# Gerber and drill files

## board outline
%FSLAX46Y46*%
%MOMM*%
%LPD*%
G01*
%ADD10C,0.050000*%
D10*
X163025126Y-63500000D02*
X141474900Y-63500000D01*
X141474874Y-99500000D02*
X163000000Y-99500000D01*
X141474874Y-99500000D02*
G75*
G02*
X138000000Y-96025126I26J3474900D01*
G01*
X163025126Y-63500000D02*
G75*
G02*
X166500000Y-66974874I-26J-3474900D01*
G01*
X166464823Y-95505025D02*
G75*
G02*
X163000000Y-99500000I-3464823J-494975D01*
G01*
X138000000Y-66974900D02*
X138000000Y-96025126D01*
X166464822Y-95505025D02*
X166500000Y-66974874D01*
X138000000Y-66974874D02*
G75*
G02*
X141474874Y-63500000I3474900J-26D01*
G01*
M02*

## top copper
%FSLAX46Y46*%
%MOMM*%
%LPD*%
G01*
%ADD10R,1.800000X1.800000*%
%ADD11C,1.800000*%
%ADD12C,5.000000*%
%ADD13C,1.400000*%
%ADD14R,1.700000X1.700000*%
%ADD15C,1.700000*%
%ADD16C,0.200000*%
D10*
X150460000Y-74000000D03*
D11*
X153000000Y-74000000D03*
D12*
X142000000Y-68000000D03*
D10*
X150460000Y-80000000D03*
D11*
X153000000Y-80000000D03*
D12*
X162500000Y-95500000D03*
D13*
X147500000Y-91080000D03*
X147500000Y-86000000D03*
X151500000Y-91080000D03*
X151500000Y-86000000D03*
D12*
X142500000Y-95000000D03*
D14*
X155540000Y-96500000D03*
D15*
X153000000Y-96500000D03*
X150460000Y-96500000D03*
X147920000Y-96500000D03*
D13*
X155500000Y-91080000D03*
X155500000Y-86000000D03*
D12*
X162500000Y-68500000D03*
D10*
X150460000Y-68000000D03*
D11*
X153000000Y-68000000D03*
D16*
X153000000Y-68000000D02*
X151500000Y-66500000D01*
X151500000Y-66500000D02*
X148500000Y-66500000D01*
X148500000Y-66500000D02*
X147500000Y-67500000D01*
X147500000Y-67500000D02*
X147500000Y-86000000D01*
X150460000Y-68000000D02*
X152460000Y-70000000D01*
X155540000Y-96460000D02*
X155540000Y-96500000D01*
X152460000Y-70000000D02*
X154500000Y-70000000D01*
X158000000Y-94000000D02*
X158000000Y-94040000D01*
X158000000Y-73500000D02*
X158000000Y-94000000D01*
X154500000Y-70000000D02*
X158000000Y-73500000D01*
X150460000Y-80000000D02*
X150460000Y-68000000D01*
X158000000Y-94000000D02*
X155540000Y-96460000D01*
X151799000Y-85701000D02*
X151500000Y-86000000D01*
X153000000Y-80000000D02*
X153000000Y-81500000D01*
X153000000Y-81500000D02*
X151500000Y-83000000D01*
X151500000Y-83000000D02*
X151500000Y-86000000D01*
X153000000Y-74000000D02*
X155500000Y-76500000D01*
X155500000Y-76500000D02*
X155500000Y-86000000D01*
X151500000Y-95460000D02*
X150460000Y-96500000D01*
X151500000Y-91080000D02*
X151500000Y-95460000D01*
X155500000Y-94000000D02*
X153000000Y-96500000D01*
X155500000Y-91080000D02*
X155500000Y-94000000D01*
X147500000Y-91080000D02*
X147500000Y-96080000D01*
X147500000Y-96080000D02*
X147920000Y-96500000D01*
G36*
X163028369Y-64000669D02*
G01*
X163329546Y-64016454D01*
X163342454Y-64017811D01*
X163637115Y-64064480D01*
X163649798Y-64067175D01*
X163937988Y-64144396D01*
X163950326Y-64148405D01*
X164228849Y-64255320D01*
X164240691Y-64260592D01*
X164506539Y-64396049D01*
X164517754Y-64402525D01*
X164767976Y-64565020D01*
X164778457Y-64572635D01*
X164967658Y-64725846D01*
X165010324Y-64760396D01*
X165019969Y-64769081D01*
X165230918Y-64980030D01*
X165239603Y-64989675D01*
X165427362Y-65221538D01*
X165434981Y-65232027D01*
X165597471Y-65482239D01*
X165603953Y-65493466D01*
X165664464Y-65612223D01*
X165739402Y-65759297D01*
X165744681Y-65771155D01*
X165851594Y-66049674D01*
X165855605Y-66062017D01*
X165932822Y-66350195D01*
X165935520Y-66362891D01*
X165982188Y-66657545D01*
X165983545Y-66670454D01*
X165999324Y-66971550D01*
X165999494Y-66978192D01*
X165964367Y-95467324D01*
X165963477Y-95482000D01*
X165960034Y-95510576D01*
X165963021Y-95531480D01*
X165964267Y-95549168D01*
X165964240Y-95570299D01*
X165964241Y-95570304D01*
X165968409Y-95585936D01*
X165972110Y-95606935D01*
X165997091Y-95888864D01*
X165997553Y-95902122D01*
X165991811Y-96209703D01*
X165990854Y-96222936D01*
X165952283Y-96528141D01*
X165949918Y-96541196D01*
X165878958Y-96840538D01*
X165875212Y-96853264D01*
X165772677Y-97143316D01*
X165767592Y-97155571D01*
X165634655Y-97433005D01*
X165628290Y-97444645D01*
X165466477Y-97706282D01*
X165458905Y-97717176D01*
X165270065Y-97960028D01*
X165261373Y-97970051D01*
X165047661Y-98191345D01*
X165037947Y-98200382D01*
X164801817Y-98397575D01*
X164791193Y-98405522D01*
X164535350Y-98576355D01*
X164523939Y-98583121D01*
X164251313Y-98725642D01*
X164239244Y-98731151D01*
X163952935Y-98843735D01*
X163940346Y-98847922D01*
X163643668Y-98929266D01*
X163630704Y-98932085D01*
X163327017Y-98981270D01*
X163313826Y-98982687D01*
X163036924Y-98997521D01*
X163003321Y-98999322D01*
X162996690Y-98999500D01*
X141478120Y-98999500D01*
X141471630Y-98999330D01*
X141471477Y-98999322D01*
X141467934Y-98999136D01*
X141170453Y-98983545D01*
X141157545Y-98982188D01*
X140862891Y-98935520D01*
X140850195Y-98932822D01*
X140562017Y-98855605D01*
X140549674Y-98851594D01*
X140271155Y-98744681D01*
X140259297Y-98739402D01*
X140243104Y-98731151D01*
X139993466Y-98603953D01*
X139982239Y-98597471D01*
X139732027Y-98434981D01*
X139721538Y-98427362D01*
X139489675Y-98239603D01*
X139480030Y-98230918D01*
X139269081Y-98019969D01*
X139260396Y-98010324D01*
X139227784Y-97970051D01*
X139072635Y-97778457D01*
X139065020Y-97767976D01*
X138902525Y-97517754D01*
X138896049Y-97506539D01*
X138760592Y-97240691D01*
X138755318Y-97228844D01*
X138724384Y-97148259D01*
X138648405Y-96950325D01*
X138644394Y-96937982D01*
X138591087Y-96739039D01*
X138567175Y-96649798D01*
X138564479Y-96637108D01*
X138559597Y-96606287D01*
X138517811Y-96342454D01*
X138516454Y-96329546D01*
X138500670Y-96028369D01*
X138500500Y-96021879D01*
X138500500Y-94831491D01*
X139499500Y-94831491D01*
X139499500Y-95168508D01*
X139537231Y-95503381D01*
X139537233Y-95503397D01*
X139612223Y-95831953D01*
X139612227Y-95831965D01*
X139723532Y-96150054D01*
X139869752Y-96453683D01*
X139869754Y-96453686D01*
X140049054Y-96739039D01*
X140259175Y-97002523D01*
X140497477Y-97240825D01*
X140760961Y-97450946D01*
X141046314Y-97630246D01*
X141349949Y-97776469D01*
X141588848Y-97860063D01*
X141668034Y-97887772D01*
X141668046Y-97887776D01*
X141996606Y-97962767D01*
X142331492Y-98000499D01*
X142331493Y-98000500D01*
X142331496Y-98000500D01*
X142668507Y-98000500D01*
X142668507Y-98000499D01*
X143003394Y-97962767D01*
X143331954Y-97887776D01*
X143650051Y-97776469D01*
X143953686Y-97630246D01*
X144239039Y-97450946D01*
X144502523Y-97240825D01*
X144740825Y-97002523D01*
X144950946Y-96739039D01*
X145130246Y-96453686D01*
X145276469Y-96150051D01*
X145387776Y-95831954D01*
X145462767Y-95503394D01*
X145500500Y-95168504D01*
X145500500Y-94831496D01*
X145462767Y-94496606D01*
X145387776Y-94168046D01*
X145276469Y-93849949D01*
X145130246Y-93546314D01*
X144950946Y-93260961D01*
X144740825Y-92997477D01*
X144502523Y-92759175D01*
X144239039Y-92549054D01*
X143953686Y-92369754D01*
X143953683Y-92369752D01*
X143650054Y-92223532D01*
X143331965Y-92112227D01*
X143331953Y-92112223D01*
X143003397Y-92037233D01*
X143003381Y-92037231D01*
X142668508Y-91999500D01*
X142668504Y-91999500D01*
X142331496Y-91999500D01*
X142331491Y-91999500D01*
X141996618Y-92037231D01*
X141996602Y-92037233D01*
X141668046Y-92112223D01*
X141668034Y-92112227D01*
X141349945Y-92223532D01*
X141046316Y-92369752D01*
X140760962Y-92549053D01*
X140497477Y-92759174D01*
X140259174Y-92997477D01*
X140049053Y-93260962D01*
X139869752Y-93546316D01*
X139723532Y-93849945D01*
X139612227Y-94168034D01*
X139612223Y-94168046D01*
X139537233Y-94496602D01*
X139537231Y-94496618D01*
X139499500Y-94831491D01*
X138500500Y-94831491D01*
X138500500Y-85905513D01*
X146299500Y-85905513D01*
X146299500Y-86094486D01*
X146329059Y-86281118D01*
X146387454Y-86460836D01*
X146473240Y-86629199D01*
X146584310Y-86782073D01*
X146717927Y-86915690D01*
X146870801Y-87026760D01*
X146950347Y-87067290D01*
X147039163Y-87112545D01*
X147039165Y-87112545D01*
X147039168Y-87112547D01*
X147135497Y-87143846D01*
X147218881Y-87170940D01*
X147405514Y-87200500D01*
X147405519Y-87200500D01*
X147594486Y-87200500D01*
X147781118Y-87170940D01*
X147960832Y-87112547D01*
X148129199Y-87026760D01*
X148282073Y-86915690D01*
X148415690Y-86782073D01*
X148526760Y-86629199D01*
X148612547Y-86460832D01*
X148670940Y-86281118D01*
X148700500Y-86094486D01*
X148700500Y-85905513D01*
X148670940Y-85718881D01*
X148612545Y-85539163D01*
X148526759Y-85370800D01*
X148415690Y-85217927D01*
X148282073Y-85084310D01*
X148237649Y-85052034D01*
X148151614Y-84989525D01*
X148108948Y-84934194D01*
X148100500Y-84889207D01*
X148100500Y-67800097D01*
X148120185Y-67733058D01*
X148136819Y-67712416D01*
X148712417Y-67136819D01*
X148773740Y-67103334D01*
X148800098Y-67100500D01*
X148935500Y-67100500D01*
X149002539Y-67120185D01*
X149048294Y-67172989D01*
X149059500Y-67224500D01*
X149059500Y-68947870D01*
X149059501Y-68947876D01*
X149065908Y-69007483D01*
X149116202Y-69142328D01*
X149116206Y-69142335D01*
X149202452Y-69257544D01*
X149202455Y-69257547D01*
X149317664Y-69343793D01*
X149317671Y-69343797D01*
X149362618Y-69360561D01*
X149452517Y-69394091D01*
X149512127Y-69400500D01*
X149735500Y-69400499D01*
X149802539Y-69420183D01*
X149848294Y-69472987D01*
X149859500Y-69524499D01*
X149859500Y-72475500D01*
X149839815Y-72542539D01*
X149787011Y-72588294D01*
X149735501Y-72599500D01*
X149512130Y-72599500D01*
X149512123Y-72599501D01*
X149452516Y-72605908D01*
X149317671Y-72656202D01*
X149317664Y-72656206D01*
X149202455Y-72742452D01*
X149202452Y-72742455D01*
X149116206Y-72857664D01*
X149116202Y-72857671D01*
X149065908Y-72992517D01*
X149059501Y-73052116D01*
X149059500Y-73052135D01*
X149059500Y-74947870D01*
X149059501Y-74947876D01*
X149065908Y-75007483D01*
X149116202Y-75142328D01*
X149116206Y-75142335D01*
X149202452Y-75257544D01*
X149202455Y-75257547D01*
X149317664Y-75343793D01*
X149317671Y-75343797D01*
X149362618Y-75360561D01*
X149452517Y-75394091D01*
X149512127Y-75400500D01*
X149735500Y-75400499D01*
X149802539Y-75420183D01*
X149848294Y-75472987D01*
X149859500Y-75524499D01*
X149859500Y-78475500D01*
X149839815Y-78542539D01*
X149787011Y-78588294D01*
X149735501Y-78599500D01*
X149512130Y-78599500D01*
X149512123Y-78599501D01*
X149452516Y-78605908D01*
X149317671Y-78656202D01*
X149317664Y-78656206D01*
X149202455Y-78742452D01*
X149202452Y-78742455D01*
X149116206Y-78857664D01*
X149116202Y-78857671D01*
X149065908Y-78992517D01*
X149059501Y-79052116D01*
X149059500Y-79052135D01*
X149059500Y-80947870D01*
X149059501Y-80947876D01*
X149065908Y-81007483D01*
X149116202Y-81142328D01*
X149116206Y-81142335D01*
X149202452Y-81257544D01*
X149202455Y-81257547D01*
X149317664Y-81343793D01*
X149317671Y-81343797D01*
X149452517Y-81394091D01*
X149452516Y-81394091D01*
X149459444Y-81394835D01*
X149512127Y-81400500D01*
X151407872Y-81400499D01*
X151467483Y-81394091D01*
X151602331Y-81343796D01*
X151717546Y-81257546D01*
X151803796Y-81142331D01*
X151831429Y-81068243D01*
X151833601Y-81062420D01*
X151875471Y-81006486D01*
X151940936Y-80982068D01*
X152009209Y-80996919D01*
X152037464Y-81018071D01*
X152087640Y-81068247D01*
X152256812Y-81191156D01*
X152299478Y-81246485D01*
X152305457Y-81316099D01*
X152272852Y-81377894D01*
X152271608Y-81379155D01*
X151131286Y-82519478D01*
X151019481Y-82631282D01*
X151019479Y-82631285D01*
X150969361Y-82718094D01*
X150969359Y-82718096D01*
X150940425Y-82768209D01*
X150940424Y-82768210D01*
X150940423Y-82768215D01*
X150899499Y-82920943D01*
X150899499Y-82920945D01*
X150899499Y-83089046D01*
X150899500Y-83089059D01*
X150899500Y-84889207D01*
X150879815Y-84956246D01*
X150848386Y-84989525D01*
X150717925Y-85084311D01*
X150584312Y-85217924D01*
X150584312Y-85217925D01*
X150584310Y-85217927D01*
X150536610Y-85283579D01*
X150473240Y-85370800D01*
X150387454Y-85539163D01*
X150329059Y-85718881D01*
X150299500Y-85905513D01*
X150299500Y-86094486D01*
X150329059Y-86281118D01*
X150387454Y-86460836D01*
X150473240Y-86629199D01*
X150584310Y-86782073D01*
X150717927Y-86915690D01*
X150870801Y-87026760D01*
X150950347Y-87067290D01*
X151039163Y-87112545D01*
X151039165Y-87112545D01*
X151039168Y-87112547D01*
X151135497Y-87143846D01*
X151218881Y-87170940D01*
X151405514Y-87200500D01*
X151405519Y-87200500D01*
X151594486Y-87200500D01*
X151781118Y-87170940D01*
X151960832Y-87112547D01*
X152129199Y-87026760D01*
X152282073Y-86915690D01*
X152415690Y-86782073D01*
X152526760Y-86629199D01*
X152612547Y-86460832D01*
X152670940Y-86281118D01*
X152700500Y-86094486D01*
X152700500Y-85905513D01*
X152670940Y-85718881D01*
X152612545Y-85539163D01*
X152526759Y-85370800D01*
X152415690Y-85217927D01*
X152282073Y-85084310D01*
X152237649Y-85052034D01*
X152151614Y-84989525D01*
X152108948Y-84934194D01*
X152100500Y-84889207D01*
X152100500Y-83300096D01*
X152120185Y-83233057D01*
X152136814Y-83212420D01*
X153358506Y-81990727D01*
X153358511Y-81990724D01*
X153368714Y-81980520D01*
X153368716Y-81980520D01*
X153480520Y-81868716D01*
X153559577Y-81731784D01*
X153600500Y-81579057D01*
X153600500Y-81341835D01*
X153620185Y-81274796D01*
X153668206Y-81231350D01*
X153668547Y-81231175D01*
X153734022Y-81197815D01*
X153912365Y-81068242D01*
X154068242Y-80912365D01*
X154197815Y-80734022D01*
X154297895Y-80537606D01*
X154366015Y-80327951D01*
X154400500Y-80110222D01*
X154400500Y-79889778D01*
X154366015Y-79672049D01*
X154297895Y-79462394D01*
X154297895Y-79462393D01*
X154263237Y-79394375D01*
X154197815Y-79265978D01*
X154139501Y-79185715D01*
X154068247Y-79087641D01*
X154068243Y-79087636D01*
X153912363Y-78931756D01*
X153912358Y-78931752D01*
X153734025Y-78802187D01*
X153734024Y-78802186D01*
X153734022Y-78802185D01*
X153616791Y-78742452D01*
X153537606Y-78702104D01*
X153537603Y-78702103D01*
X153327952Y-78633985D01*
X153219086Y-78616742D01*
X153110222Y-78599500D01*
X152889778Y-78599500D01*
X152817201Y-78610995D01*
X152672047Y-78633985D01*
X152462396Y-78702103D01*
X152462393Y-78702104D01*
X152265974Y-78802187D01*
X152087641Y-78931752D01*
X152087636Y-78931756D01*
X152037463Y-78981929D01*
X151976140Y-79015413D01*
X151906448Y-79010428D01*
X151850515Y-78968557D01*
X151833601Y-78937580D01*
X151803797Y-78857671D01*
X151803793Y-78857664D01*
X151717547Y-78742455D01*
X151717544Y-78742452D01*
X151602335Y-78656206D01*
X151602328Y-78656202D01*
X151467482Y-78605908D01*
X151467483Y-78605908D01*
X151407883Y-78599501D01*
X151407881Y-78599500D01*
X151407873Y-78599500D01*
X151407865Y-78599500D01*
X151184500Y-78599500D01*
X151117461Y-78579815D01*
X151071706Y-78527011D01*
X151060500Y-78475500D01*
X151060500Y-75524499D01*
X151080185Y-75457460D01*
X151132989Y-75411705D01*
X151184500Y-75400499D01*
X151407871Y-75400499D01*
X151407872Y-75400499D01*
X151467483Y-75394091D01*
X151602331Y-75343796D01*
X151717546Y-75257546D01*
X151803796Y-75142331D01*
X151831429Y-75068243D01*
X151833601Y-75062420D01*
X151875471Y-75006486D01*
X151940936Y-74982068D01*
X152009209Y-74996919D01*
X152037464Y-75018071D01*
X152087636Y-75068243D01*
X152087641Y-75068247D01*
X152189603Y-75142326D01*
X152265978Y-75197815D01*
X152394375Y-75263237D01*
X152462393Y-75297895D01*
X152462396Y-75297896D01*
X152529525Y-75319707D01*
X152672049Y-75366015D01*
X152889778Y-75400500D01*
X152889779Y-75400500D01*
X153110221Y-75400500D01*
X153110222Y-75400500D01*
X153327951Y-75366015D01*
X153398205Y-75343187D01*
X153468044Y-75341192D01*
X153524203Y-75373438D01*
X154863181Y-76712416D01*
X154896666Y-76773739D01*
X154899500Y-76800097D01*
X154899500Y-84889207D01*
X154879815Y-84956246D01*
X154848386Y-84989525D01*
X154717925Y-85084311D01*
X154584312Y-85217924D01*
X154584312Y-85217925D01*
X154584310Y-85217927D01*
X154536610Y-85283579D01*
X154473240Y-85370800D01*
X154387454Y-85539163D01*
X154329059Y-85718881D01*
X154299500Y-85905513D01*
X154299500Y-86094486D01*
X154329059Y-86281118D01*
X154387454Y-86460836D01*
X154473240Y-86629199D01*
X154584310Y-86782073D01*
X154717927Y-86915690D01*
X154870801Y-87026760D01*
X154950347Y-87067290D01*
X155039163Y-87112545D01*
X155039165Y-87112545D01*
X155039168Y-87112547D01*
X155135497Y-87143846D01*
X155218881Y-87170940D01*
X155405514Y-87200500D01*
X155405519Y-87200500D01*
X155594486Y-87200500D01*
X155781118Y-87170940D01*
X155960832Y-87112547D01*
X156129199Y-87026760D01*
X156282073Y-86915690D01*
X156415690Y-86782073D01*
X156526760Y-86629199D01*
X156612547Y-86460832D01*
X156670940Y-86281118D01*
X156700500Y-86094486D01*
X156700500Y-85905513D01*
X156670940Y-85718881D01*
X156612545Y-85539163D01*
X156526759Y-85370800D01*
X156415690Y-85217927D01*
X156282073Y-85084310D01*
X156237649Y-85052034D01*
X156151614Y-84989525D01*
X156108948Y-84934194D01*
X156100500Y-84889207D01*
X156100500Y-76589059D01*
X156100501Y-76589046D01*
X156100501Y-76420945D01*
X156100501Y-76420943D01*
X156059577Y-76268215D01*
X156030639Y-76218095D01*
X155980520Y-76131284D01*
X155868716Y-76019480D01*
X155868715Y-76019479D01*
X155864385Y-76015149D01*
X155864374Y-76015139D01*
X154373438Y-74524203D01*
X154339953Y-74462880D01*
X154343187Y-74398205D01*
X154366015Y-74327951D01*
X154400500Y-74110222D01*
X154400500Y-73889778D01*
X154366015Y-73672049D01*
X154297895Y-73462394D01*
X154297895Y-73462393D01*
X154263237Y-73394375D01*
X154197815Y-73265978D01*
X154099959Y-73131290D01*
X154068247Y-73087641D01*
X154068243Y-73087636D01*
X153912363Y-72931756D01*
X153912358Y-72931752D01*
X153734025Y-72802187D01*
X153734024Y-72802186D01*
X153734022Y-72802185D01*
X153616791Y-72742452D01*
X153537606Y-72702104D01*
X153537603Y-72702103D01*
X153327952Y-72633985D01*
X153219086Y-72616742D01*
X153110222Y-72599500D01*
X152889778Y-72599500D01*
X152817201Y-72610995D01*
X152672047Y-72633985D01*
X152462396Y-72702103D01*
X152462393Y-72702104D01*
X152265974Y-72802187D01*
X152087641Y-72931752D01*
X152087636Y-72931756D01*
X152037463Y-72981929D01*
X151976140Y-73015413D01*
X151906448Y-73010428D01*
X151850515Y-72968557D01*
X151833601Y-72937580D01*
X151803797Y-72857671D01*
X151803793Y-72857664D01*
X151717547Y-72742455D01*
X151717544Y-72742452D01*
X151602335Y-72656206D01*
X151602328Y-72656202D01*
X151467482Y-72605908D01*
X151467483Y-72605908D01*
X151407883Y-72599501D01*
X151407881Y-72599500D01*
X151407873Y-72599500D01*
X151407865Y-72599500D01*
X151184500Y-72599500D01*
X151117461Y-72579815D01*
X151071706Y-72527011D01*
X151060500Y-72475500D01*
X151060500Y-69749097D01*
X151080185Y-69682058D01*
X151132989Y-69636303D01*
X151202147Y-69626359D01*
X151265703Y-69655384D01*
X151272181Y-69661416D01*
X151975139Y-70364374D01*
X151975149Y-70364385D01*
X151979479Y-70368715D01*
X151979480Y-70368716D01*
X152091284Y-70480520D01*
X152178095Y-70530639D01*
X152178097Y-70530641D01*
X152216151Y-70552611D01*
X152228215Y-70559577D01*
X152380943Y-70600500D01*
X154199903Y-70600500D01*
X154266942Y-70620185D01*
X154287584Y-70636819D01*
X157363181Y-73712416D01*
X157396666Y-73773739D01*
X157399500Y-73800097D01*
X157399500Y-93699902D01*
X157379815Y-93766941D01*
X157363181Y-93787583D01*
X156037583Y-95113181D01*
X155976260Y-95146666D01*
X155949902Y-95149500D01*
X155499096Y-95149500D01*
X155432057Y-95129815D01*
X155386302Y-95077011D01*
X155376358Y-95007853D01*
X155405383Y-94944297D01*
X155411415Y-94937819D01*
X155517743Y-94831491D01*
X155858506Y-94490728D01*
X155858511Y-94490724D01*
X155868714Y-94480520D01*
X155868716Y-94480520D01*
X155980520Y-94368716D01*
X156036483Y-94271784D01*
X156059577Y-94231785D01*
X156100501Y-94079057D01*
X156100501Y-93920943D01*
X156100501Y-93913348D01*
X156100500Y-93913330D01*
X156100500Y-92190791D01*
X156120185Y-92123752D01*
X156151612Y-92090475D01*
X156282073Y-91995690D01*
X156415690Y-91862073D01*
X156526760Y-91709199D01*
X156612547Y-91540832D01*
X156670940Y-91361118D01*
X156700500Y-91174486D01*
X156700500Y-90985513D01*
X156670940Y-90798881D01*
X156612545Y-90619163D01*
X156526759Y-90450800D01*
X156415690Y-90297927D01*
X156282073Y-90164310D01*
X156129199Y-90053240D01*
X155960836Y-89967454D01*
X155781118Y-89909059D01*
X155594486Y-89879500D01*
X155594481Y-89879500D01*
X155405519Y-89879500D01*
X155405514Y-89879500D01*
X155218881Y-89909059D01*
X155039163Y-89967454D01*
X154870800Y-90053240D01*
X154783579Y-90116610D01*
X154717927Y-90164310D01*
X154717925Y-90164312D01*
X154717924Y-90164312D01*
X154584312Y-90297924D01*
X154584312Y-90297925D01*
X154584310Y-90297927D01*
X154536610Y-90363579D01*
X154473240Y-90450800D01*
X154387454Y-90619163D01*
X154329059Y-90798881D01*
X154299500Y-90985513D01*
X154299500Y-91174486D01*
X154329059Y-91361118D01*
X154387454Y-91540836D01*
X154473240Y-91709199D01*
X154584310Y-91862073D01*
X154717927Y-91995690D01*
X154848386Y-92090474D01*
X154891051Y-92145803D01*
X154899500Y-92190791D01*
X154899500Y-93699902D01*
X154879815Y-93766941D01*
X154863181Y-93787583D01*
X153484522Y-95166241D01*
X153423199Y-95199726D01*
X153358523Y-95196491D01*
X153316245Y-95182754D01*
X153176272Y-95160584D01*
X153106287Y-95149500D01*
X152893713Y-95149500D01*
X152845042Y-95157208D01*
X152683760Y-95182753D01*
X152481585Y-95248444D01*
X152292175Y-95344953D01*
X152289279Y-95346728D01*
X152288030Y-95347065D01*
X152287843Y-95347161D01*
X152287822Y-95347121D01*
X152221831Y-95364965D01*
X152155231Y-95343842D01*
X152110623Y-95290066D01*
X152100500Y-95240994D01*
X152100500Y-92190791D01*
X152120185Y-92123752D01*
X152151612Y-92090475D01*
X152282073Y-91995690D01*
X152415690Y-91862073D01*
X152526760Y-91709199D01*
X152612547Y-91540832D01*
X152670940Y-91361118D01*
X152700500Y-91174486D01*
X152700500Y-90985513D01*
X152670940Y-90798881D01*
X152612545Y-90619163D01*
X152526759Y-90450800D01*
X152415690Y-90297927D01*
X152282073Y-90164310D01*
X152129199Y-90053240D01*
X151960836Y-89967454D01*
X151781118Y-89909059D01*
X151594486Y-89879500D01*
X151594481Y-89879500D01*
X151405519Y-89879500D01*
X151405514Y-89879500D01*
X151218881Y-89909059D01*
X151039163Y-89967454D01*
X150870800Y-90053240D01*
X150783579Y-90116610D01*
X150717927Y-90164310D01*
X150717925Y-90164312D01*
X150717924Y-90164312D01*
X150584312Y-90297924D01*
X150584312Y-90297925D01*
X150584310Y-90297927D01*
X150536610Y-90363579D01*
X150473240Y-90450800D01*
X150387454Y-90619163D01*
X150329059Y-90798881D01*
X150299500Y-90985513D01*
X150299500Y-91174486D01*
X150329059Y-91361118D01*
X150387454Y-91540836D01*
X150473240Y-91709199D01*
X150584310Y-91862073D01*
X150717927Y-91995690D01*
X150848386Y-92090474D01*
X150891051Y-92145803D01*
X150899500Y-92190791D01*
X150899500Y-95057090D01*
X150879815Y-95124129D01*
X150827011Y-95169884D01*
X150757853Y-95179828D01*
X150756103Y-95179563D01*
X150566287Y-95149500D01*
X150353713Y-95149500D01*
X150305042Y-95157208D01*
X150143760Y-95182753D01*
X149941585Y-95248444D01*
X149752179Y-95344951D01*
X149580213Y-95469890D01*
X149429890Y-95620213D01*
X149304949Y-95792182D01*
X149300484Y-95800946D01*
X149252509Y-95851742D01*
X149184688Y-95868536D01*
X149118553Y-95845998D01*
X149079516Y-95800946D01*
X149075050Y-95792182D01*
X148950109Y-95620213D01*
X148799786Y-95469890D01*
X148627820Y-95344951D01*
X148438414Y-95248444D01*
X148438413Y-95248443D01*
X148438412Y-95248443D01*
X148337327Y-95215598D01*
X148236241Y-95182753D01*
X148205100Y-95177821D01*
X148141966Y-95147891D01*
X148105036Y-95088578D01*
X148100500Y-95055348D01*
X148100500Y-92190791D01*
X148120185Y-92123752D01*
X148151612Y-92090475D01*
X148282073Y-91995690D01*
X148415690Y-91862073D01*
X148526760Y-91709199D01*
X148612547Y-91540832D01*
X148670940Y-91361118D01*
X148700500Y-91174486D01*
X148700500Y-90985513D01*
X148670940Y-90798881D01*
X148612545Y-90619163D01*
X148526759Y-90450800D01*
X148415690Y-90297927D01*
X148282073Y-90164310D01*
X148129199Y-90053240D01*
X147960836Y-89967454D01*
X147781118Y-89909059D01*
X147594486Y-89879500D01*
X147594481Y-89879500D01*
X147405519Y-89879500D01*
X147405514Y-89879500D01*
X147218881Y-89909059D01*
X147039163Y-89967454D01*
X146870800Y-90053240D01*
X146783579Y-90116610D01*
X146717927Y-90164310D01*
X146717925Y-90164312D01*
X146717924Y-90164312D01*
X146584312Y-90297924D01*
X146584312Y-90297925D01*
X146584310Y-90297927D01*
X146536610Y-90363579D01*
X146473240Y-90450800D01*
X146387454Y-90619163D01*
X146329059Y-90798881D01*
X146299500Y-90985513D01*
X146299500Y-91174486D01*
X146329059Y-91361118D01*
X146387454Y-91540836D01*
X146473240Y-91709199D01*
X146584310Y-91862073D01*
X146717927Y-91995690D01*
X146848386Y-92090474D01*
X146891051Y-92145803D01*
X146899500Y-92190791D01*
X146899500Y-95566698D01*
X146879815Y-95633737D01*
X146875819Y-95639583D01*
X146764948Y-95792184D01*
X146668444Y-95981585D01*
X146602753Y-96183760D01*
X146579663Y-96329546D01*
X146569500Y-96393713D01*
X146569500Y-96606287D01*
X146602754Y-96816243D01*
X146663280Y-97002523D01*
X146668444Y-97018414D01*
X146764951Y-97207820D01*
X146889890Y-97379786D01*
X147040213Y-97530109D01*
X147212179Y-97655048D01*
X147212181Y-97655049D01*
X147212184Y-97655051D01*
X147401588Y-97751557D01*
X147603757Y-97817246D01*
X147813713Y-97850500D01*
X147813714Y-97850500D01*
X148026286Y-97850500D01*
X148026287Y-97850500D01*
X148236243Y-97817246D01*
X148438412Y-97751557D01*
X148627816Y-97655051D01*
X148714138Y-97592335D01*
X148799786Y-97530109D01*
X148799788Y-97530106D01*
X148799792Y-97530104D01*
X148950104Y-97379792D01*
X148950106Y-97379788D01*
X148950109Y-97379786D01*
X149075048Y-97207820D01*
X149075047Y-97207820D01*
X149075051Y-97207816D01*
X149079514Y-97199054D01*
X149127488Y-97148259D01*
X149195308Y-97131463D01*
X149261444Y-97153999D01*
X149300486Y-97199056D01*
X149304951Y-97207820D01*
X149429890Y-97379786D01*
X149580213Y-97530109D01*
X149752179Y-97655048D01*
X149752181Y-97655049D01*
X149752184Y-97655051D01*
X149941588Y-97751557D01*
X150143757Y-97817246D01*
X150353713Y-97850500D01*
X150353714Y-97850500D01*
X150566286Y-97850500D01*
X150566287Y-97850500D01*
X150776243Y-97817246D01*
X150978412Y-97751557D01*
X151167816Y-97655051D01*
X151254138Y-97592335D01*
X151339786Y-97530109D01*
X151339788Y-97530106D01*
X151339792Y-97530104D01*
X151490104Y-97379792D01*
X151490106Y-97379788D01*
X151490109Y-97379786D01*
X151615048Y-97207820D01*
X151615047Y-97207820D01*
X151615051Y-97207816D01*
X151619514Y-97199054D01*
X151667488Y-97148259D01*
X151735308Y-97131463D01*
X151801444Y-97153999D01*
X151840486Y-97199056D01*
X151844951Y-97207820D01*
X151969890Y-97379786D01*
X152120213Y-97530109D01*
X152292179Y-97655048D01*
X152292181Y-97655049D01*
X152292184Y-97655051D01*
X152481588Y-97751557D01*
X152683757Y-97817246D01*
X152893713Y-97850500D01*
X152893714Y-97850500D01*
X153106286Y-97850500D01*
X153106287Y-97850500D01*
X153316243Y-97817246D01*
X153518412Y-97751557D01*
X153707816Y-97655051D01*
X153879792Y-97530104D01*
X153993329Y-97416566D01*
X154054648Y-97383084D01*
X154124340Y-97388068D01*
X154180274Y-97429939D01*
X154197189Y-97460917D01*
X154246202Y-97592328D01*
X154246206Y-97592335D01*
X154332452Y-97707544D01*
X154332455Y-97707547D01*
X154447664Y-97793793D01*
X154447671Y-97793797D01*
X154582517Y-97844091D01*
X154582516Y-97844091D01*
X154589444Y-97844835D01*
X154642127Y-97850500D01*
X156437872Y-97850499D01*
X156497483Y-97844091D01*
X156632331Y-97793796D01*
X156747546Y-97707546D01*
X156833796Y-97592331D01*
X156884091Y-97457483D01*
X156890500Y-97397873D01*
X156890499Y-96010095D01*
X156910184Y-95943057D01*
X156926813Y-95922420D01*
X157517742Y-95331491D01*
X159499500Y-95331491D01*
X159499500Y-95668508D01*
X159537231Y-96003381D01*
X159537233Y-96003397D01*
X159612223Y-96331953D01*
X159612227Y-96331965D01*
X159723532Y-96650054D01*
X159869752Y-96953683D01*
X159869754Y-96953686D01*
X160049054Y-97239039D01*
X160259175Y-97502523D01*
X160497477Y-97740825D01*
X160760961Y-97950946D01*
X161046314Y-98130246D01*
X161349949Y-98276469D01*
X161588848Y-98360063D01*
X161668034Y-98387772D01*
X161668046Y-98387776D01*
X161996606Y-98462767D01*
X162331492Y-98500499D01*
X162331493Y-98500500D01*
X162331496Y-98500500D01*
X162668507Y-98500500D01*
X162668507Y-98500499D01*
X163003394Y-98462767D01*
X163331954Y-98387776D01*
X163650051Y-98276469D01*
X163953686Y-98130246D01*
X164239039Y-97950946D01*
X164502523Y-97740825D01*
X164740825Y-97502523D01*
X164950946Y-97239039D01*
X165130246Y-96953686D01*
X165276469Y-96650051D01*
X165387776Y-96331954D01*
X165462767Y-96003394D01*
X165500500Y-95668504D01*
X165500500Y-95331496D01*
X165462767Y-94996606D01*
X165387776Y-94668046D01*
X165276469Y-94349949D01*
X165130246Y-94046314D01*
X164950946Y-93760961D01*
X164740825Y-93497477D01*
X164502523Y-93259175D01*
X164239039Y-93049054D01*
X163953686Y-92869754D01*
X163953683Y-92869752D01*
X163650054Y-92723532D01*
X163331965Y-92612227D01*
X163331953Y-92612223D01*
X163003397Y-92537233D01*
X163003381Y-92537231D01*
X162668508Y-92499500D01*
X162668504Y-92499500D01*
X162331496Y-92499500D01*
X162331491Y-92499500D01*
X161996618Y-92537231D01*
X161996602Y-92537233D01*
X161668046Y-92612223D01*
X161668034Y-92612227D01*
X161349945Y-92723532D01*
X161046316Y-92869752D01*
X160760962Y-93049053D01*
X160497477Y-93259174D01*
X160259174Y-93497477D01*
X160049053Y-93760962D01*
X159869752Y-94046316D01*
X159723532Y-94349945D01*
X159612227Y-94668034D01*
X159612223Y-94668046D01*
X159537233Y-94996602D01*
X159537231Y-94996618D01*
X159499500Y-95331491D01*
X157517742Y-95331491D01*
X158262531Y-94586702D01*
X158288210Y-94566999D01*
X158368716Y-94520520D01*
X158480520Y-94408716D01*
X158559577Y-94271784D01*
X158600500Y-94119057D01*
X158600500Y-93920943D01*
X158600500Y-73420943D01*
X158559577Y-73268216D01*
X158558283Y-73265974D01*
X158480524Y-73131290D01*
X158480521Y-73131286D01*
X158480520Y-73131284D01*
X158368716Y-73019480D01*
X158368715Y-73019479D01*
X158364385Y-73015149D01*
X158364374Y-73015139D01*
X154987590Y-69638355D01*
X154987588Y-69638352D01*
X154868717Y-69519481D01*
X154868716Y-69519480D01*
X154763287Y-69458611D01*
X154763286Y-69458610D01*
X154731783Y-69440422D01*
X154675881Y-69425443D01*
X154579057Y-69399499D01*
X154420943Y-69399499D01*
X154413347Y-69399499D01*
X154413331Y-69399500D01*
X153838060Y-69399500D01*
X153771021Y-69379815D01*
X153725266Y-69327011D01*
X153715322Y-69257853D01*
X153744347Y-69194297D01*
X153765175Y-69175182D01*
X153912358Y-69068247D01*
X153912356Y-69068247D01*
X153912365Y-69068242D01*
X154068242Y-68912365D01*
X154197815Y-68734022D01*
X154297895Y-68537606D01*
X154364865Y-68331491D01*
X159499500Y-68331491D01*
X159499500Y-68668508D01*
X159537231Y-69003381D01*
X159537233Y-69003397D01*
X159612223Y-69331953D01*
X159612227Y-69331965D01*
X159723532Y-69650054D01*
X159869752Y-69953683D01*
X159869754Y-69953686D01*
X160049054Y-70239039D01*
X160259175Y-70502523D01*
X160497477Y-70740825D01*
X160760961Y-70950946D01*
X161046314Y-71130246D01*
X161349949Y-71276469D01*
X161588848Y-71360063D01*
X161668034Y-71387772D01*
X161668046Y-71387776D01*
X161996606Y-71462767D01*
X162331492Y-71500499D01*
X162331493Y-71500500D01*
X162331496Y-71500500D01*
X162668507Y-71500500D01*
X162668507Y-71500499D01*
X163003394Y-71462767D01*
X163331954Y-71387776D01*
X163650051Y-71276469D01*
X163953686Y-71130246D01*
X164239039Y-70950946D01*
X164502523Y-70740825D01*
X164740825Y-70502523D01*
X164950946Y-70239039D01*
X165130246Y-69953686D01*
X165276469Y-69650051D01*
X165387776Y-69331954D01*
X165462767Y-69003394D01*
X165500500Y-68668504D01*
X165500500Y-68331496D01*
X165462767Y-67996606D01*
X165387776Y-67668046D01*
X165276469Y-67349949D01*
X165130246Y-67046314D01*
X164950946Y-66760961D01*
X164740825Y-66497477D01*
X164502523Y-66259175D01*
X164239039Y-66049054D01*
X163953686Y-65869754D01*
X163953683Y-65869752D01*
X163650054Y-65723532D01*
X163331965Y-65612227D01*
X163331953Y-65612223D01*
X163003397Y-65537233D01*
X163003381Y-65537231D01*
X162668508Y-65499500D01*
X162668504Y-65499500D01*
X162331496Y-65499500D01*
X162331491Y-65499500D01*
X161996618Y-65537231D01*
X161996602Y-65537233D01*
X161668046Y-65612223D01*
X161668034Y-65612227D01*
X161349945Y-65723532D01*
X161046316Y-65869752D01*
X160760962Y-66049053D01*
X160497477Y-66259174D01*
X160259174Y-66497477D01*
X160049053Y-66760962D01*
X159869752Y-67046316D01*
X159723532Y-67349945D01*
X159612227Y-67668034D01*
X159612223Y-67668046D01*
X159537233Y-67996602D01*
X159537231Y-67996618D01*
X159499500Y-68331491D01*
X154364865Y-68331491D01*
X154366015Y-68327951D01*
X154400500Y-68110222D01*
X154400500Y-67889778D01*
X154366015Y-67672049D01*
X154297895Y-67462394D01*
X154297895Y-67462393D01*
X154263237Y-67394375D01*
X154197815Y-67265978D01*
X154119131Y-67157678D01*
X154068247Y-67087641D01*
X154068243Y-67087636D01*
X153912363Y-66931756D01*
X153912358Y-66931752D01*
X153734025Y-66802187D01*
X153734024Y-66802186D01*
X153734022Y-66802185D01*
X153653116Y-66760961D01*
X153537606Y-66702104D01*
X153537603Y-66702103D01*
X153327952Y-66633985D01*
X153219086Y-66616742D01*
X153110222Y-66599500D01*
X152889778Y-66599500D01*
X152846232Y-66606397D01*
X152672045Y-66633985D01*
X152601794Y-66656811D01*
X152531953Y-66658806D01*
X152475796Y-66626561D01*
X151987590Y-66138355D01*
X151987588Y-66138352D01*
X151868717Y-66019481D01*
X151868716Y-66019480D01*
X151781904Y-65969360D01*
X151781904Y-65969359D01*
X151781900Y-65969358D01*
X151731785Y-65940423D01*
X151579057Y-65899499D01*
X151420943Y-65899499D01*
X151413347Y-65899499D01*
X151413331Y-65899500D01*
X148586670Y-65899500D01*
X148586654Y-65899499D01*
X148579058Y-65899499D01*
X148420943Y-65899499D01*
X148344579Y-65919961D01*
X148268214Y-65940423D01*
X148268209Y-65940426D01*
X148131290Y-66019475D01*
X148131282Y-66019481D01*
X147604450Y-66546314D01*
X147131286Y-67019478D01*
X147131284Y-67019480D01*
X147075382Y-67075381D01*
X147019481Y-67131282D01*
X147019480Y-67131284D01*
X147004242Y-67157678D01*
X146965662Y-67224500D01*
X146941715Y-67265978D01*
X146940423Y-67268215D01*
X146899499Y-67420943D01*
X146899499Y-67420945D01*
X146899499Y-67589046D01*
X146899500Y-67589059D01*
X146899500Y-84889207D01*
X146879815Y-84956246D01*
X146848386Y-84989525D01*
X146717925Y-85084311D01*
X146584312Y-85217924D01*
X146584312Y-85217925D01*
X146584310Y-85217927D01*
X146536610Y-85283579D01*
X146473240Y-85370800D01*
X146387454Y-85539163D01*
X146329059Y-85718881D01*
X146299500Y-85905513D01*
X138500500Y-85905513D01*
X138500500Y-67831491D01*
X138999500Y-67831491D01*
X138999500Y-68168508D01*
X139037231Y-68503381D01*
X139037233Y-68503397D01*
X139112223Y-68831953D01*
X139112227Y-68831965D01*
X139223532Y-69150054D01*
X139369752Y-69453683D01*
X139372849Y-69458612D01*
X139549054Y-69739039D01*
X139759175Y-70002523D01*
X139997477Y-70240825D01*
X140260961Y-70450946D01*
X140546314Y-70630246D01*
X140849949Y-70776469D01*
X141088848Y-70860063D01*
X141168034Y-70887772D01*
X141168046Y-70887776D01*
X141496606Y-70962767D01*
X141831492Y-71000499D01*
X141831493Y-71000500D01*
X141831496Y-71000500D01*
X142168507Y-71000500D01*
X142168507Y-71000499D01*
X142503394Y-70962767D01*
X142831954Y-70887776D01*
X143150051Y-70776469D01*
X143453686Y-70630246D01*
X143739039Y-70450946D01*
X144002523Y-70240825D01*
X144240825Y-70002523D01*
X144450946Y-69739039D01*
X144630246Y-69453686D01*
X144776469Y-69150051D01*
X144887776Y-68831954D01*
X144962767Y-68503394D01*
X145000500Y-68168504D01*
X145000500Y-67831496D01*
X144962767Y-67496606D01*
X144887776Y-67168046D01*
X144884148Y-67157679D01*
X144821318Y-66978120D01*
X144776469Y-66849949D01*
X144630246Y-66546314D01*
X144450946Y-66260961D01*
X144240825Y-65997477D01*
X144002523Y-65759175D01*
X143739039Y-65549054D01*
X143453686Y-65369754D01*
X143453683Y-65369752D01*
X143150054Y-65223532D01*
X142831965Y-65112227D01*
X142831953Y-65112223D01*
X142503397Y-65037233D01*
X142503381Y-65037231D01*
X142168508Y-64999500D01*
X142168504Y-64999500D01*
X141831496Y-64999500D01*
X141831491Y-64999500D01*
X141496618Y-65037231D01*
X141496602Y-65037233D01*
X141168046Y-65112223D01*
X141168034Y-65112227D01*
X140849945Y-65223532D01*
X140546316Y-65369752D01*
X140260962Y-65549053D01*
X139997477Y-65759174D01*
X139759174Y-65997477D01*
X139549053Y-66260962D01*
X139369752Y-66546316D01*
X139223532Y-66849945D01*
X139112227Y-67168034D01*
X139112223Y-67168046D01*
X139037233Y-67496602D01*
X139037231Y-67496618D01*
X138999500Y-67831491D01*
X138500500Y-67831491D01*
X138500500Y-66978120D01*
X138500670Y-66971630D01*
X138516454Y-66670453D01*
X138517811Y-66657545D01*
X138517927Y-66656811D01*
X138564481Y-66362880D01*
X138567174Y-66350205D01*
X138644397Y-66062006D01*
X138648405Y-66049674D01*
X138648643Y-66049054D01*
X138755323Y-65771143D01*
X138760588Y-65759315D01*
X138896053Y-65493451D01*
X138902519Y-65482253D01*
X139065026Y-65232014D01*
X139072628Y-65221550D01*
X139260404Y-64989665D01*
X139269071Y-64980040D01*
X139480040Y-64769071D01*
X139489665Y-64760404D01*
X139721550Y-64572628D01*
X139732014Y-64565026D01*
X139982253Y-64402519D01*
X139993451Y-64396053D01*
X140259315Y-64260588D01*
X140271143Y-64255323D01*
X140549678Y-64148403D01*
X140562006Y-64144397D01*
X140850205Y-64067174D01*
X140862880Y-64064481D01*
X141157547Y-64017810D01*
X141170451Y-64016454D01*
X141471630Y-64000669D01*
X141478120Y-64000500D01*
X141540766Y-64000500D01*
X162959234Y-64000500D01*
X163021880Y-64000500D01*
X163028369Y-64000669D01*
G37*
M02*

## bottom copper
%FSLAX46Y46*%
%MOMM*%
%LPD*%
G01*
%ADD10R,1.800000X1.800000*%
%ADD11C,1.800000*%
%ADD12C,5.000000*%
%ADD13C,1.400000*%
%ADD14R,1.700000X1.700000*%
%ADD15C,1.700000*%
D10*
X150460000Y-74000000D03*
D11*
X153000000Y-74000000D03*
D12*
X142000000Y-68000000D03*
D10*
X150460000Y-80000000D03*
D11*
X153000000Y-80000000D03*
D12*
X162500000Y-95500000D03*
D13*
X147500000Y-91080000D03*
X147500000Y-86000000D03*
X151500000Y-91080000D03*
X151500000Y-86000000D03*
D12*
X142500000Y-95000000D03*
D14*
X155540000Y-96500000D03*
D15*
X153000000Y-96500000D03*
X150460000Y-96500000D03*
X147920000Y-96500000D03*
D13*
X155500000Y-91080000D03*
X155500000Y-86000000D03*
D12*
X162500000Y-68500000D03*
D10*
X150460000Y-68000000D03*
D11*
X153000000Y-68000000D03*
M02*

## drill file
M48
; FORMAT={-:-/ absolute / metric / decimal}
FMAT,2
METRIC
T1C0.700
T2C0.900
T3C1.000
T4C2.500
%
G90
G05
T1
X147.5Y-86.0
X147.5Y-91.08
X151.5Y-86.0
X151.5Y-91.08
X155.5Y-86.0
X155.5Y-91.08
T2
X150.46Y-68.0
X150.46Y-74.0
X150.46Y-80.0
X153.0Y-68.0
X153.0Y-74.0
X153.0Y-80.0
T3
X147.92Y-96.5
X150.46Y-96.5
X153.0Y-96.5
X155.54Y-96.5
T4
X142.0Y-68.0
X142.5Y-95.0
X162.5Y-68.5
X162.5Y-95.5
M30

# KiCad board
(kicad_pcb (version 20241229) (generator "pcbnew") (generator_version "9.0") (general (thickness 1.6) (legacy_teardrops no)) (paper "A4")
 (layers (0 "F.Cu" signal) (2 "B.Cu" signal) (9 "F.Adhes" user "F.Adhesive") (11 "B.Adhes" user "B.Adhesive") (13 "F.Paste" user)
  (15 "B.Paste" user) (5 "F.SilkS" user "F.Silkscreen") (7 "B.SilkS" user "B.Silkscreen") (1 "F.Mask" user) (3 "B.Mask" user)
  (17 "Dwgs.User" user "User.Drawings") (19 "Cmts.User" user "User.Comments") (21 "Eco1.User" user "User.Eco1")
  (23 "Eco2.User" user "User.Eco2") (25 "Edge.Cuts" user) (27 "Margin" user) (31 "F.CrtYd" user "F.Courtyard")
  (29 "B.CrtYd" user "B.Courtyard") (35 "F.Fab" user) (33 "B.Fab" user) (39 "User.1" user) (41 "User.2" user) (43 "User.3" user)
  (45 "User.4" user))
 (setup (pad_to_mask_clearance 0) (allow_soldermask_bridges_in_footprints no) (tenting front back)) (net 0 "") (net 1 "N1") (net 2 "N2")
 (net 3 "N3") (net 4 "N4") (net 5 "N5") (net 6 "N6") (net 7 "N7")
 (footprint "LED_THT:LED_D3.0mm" (layer "F.Cu") (at 150.46 74)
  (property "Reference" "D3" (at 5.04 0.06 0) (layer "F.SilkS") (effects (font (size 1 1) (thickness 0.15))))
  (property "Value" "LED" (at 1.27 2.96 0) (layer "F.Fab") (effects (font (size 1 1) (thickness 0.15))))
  (pad "1" thru_hole rect (at 0 0) (size 1.8 1.8) (drill 0.9) (layers "*.Cu" "*.Mask") (remove_unused_layers no) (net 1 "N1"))
  (pad "2" thru_hole circle (at 2.54 0) (size 1.8 1.8) (drill 0.9) (layers "*.Cu" "*.Mask") (remove_unused_layers no) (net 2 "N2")))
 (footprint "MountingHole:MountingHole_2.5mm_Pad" (layer "F.Cu") (at 142 68)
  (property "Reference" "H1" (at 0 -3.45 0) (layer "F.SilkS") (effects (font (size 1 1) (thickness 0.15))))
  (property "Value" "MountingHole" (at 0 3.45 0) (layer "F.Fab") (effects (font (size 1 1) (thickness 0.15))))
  (pad "1" thru_hole circle (at 0 0) (size 5 5) (drill 2.5) (layers "*.Cu" "*.Mask") (remove_unused_layers no) (zone_connect 2)))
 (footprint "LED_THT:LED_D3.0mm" (layer "F.Cu") (at 150.46 80)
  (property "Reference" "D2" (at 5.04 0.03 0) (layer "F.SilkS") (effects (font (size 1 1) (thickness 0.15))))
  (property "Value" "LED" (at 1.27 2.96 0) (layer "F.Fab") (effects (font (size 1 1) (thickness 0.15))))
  (pad "1" thru_hole rect (at 0 0) (size 1.8 1.8) (drill 0.9) (layers "*.Cu" "*.Mask") (remove_unused_layers no) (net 1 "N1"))
  (pad "2" thru_hole circle (at 2.54 0) (size 1.8 1.8) (drill 0.9) (layers "*.Cu" "*.Mask") (remove_unused_layers no) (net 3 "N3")))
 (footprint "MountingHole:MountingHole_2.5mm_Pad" (layer "F.Cu") (at 162.5 95.5)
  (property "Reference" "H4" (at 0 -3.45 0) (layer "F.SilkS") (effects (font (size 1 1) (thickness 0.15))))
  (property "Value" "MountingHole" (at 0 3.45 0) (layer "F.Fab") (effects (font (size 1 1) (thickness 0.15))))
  (pad "1" thru_hole circle (at 0 0) (size 5 5) (drill 2.5) (layers "*.Cu" "*.Mask") (remove_unused_layers no) (zone_connect 2)))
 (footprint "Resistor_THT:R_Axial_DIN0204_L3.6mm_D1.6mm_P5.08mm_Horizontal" (layer "F.Cu") (at 147.5 91.08 90)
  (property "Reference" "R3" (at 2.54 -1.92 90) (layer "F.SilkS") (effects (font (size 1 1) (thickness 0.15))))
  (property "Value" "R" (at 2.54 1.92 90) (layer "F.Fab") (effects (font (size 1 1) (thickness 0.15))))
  (pad "1" thru_hole circle (at 0 0 90) (size 1.4 1.4) (drill 0.7) (layers "*.Cu" "*.Mask") (remove_unused_layers no) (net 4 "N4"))
  (pad "2" thru_hole circle (at 5.08 0 90) (size 1.4 1.4) (drill 0.7) (layers "*.Cu" "*.Mask") (remove_unused_layers no) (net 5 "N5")))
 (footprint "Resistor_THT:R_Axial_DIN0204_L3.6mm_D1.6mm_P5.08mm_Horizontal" (layer "F.Cu") (at 151.5 91.08 90)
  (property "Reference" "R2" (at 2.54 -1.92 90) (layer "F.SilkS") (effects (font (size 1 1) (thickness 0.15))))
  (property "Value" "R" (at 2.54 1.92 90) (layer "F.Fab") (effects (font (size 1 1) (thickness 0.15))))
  (pad "1" thru_hole circle (at 0 0 90) (size 1.4 1.4) (drill 0.7) (layers "*.Cu" "*.Mask") (remove_unused_layers no) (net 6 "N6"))
  (pad "2" thru_hole circle (at 5.08 0 90) (size 1.4 1.4) (drill 0.7) (layers "*.Cu" "*.Mask") (remove_unused_layers no) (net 3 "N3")))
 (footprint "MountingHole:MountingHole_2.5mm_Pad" (layer "F.Cu") (at 142.5 95)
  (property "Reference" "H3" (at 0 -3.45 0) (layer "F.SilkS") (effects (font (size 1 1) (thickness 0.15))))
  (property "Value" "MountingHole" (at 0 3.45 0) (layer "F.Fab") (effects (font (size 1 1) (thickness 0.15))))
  (pad "1" thru_hole circle (at 0 0) (size 5 5) (drill 2.5) (layers "*.Cu" "*.Mask") (remove_unused_layers no) (zone_connect 2)))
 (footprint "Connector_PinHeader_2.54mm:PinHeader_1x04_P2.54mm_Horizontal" (layer "F.Cu") (at 155.54 96.5 -90)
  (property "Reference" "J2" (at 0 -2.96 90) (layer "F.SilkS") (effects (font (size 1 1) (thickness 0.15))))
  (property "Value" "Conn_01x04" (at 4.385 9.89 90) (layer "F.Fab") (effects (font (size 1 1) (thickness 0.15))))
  (pad "1" thru_hole rect (at 0 0 270) (size 1.7 1.7) (drill 1) (layers "*.Cu" "*.Mask") (remove_unused_layers no) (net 1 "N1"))
  (pad "2" thru_hole circle (at 0 2.54 270) (size 1.7 1.7) (drill 1) (layers "*.Cu" "*.Mask") (remove_unused_layers no) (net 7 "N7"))
  (pad "3" thru_hole circle (at 0 5.08 270) (size 1.7 1.7) (drill 1) (layers "*.Cu" "*.Mask") (remove_unused_layers no) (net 6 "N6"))
  (pad "4" thru_hole circle (at 0 7.62 270) (size 1.7 1.7) (drill 1) (layers "*.Cu" "*.Mask") (remove_unused_layers no) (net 4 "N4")))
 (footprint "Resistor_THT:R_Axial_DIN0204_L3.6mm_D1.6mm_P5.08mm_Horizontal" (layer "F.Cu") (at 155.5 91.08 90)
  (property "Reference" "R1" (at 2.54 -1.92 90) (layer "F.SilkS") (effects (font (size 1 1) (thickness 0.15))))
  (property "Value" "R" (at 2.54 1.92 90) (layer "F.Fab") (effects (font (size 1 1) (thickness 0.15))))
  (pad "1" thru_hole circle (at 0 0 90) (size 1.4 1.4) (drill 0.7) (layers "*.Cu" "*.Mask") (remove_unused_layers no) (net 7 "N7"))
  (pad "2" thru_hole circle (at 5.08 0 90) (size 1.4 1.4) (drill 0.7) (layers "*.Cu" "*.Mask") (remove_unused_layers no) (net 2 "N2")))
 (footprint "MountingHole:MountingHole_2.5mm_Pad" (layer "F.Cu") (at 162.5 68.5)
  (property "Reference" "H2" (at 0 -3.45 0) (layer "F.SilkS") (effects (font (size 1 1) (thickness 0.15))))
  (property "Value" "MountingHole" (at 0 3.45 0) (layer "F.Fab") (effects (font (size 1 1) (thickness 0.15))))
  (pad "1" thru_hole circle (at 0 0) (size 5 5) (drill 2.5) (layers "*.Cu" "*.Mask") (remove_unused_layers no) (zone_connect 2)))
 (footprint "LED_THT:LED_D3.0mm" (layer "F.Cu") (at 150.46 68)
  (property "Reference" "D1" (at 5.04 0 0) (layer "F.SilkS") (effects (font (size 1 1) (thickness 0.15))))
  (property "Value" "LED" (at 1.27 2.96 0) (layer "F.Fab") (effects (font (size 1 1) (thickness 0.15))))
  (pad "1" thru_hole rect (at 0 0) (size 1.8 1.8) (drill 0.9) (layers "*.Cu" "*.Mask") (remove_unused_layers no) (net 1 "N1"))
  (pad "2" thru_hole circle (at 2.54 0) (size 1.8 1.8) (drill 0.9) (layers "*.Cu" "*.Mask") (remove_unused_layers no) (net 5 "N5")))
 (gr_line (start 163.025126 63.5) (end 141.4749 63.5) (stroke (width 0.05) (type default)) (layer "Edge.Cuts"))
 (gr_line (start 141.474874 99.5) (end 163 99.5) (stroke (width 0.05) (type default)) (layer "Edge.Cuts"))
 (gr_arc (start 141.474874 99.5) (mid 139.017767 98.482233) (end 138 96.025126) (stroke (width 0.05) (type default)) (layer "Edge.Cuts"))
 (gr_arc (start 163.025126 63.5) (mid 165.482233 64.517767) (end 166.5 66.974874) (stroke (width 0.05) (type default)) (layer "Edge.Cuts"))
 (gr_arc (start 166.464823 95.505025) (mid 165.644089 98.293206) (end 163 99.5) (stroke (width 0.05) (type default)) (layer "Edge.Cuts"))
 (gr_line (start 138 66.9749) (end 138 96.025126) (stroke (width 0.05) (type default)) (layer "Edge.Cuts"))
 (gr_line (start 166.464822 95.505025) (end 166.5 66.974874) (stroke (width 0.05) (type default)) (layer "Edge.Cuts"))
 (gr_arc (start 138 66.974874) (mid 139.017767 64.517767) (end 141.474874 63.5) (stroke (width 0.05) (type default)) (layer "Edge.Cuts"))
 (segment (start 153 68) (end 151.5 66.5) (width 0.2) (layer "F.Cu") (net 5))
 (segment (start 151.5 66.5) (end 148.5 66.5) (width 0.2) (layer "F.Cu") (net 5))
 (segment (start 148.5 66.5) (end 147.5 67.5) (width 0.2) (layer "F.Cu") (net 5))
 (segment (start 147.5 67.5) (end 147.5 86) (width 0.2) (layer "F.Cu") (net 5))
 (segment (start 150.46 68) (end 152.46 70) (width 0.2) (layer "F.Cu") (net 1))
 (segment (start 155.54 96.46) (end 155.54 96.5) (width 0.2) (layer "F.Cu") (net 1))
 (segment (start 152.46 70) (end 154.5 70) (width 0.2) (layer "F.Cu") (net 1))
 (segment (start 158 94) (end 158 94.04) (width 0.2) (layer "F.Cu") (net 1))
 (segment (start 158 73.5) (end 158 94) (width 0.2) (layer "F.Cu") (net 1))
 (segment (start 154.5 70) (end 158 73.5) (width 0.2) (layer "F.Cu") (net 1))
 (segment (start 150.46 80) (end 150.46 68) (width 0.2) (layer "F.Cu") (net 1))
 (segment (start 158 94) (end 155.54 96.46) (width 0.2) (layer "F.Cu") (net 1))
 (segment (start 151.799 85.701) (end 151.5 86) (width 0.2) (layer "F.Cu") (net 3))
 (segment (start 153 80) (end 153 81.5) (width 0.2) (layer "F.Cu") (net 3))
 (segment (start 153 81.5) (end 151.5 83) (width 0.2) (layer "F.Cu") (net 3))
 (segment (start 151.5 83) (end 151.5 86) (width 0.2) (layer "F.Cu") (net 3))
 (segment (start 153 74) (end 155.5 76.5) (width 0.2) (layer "F.Cu") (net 2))
 (segment (start 155.5 76.5) (end 155.5 86) (width 0.2) (layer "F.Cu") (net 2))
 (segment (start 151.5 95.46) (end 150.46 96.5) (width 0.2) (layer "F.Cu") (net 6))
 (segment (start 151.5 91.08) (end 151.5 95.46) (width 0.2) (layer "F.Cu") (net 6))
 (segment (start 155.5 94) (end 153 96.5) (width 0.2) (layer "F.Cu") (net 7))
 (segment (start 155.5 91.08) (end 155.5 94) (width 0.2) (layer "F.Cu") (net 7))
 (segment (start 147.5 91.08) (end 147.5 96.08) (width 0.2) (layer "F.Cu") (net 4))
 (segment (start 147.5 96.08) (end 147.92 96.5) (width 0.2) (layer "F.Cu") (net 4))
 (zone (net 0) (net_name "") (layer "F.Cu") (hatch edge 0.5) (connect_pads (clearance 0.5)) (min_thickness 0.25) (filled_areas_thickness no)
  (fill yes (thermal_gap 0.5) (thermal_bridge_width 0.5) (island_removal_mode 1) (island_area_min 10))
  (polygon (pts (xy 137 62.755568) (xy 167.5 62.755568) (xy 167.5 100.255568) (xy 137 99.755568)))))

